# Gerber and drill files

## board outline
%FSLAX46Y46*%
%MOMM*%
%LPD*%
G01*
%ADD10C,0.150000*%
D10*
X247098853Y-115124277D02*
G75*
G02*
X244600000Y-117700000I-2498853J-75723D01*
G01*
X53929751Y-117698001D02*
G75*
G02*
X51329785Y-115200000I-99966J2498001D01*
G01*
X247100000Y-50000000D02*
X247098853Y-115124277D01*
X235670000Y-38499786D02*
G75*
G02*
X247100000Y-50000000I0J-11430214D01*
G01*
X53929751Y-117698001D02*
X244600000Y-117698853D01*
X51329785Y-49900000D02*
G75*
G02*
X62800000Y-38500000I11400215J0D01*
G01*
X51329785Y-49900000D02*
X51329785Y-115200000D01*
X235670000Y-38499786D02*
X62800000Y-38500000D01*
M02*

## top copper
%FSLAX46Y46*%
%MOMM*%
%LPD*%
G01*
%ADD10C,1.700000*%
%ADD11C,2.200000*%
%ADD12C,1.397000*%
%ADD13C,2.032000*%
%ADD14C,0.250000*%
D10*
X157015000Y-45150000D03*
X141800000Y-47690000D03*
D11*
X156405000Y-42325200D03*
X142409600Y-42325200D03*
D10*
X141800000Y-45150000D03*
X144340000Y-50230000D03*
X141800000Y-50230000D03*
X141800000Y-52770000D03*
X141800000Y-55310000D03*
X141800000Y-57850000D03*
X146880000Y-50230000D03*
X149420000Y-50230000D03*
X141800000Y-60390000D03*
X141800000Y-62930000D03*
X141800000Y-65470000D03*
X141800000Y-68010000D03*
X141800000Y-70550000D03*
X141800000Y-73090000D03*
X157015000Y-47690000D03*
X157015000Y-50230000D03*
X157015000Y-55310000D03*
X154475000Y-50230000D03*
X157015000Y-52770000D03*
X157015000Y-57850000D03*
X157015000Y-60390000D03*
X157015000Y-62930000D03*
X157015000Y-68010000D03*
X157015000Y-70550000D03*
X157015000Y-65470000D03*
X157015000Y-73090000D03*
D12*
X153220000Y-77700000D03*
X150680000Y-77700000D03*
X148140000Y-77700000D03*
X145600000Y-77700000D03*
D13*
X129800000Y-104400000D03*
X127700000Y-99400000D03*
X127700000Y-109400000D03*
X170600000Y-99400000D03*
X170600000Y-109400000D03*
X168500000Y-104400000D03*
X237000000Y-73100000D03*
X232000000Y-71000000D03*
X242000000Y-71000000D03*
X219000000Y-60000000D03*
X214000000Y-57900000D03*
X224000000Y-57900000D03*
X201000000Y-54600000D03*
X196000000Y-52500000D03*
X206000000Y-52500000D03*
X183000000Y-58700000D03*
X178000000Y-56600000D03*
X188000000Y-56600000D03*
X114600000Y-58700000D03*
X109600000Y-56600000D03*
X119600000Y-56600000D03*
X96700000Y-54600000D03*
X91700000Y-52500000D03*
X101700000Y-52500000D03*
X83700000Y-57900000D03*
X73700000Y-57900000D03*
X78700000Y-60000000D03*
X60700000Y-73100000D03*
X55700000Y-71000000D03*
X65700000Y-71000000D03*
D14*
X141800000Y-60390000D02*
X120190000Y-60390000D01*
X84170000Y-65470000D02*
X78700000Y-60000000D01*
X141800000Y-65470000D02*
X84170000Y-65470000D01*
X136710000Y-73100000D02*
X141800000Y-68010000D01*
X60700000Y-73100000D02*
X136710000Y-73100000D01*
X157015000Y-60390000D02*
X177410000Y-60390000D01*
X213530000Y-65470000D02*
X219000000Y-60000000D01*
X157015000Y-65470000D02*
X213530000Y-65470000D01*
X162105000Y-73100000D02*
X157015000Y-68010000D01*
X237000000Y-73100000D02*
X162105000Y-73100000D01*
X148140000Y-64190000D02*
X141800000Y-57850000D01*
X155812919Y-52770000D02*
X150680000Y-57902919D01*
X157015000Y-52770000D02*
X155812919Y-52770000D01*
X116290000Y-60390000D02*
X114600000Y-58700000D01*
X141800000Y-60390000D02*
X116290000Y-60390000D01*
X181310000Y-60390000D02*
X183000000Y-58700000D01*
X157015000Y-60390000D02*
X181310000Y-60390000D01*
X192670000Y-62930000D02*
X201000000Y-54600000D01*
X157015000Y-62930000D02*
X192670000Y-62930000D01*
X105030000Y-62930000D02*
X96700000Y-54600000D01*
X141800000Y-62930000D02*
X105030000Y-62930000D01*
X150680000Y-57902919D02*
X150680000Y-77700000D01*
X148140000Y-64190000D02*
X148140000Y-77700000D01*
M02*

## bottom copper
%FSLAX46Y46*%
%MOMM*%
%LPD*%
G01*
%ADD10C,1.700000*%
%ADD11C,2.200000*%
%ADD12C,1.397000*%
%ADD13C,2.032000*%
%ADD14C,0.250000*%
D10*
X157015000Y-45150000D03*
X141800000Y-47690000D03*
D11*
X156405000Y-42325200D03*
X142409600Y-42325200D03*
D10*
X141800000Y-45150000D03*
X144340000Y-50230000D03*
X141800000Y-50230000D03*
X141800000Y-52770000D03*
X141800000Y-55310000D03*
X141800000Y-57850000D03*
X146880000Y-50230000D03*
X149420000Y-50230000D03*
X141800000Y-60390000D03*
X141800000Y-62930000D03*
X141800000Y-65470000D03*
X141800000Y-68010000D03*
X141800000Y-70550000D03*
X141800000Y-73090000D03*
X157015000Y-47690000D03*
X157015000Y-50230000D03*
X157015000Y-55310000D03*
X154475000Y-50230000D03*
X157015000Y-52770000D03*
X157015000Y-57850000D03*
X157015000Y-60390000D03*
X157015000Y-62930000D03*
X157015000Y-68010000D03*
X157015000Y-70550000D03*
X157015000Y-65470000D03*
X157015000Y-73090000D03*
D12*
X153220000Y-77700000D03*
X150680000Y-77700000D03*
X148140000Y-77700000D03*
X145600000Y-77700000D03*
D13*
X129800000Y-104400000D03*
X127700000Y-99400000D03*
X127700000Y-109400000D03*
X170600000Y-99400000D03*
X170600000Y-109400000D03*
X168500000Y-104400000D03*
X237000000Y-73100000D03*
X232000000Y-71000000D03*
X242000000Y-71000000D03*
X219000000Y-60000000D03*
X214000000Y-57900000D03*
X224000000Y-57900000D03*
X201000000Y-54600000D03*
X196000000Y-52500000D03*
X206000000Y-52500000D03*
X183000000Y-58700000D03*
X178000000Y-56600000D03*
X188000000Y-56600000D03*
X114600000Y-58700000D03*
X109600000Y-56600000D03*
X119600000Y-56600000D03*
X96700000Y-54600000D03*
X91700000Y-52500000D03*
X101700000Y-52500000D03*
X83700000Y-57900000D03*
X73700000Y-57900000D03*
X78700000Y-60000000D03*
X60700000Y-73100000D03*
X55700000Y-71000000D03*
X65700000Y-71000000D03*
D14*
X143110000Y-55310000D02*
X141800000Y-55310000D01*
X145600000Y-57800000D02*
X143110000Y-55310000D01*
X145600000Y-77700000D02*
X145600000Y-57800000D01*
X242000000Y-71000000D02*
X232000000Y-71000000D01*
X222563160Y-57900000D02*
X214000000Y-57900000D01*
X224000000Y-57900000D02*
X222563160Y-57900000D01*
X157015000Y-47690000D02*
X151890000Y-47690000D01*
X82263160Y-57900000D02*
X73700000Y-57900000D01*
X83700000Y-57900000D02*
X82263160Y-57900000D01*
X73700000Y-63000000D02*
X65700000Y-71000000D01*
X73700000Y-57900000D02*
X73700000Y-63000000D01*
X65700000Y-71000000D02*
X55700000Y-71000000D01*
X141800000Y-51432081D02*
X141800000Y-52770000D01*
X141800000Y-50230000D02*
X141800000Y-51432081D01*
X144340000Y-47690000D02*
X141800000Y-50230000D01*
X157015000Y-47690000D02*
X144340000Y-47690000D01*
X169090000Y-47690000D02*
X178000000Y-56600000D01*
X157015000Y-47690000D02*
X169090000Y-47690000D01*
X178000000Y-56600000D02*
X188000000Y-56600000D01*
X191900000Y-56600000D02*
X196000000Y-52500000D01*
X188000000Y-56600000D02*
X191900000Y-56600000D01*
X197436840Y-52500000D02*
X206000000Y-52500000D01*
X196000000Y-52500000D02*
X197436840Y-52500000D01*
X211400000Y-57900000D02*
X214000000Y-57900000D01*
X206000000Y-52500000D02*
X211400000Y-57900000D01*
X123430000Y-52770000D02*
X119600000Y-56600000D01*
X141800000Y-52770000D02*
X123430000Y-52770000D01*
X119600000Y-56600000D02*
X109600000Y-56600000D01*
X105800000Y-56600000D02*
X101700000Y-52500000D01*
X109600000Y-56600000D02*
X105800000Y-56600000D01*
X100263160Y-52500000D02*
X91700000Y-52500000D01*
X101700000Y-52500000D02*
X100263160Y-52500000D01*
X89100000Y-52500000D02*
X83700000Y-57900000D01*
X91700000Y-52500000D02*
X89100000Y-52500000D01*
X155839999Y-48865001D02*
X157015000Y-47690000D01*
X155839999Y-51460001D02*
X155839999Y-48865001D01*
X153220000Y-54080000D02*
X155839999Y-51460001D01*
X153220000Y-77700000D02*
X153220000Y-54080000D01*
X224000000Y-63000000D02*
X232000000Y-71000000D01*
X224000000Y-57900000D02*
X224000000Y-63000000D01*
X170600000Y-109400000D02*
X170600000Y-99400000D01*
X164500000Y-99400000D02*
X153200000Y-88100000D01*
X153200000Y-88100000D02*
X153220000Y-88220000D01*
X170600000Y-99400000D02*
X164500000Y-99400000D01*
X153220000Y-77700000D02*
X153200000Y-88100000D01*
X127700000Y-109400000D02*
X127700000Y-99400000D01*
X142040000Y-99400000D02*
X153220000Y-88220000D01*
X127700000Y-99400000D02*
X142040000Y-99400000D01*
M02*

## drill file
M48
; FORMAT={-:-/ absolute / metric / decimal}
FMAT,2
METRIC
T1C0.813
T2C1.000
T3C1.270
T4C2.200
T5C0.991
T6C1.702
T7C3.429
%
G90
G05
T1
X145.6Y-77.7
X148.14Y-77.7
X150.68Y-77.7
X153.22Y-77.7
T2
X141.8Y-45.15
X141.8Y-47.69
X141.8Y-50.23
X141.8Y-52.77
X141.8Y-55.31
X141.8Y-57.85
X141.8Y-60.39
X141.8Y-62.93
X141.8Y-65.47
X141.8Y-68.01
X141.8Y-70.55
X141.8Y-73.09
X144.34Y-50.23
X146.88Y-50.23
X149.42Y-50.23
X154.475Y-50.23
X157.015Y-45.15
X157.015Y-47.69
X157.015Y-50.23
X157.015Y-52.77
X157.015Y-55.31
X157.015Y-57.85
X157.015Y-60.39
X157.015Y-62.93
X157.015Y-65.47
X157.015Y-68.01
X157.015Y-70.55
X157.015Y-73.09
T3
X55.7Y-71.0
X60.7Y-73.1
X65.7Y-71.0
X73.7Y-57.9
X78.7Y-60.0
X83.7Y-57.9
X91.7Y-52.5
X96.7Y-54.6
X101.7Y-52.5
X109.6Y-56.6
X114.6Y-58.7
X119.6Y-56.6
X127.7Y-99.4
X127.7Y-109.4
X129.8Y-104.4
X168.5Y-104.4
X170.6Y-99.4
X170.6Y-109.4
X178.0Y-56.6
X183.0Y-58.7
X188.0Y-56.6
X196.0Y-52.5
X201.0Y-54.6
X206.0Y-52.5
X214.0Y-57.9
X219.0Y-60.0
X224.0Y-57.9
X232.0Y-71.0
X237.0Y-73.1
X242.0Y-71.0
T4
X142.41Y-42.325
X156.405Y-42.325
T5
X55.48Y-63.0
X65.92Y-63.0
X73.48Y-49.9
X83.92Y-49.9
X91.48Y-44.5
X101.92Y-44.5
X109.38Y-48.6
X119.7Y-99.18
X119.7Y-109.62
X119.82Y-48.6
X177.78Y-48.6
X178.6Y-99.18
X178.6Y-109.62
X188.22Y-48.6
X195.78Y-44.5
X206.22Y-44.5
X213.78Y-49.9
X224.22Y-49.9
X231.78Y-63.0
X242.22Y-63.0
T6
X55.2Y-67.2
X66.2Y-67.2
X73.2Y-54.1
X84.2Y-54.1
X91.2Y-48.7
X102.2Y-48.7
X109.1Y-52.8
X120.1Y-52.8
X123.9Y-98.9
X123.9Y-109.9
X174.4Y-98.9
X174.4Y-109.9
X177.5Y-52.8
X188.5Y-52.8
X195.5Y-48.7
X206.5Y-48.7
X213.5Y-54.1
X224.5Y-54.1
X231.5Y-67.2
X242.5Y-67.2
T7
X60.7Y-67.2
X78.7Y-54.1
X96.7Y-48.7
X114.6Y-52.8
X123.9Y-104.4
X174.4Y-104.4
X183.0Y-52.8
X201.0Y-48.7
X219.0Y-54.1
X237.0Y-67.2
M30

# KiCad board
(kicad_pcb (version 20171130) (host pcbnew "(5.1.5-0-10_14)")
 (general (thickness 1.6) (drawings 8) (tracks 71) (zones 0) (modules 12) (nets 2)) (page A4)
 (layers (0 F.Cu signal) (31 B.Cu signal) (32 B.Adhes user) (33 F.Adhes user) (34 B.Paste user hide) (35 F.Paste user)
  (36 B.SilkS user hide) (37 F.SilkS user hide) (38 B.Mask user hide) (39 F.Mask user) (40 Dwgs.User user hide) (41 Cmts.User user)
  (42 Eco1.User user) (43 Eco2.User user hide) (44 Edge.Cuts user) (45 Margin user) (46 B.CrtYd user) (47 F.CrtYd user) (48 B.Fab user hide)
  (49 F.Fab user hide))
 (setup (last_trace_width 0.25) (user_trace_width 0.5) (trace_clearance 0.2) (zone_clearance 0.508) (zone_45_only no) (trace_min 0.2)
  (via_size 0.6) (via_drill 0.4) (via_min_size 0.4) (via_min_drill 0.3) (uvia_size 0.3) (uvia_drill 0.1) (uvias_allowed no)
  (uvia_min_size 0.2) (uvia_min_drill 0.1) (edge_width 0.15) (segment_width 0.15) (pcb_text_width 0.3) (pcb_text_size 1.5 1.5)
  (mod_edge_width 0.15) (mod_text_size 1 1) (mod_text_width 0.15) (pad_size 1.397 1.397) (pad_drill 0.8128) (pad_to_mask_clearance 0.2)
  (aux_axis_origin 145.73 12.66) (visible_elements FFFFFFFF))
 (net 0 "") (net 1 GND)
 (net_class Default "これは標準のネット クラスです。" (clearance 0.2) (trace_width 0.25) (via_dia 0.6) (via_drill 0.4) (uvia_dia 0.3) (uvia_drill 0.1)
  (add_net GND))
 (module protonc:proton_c (layer F.Cu) (at 149.4 60.4)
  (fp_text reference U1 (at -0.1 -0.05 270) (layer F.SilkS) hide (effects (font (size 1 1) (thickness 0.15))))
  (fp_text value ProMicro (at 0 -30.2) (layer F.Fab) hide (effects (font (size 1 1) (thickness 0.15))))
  (pad 5V thru_hole circle (at 7.615 -15.25) (size 1.7 1.7) (drill 1) (layers *.Cu *.Mask))
  (pad A10 thru_hole circle (at -7.6 -12.71) (size 1.7 1.7) (drill 1) (layers *.Cu *.Mask))
  (pad SCRE thru_hole circle (at 7.005 -18.0748) (size 2.2 2.2) (drill 2.2) (layers *.Cu *.Mask))
  (pad SCRE thru_hole circle (at -6.9904 -18.0748) (size 2.2 2.2) (drill 2.2) (layers *.Cu *.Mask))
  (pad A9 thru_hole circle (at -7.6 -15.25) (size 1.7 1.7) (drill 1) (layers *.Cu *.Mask))
  (pad D+ thru_hole circle (at -5.06 -10.17) (size 1.7 1.7) (drill 1) (layers *.Cu *.Mask))
  (pad GND thru_hole circle (at -7.6 -10.17) (size 1.7 1.7) (drill 1) (layers *.Cu *.Mask) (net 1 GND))
  (pad GND thru_hole circle (at -7.6 -7.63) (size 1.7 1.7) (drill 1) (layers *.Cu *.Mask) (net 1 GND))
  (pad B7 thru_hole circle (at -7.6 -5.09) (size 1.7 1.7) (drill 1) (layers *.Cu *.Mask))
  (pad B6 thru_hole circle (at -7.6 -2.55) (size 1.7 1.7) (drill 1) (layers *.Cu *.Mask))
  (pad D- thru_hole circle (at -2.52 -10.17) (size 1.7 1.7) (drill 1) (layers *.Cu *.Mask))
  (pad CHRG thru_hole circle (at 0.02 -10.17) (size 1.7 1.7) (drill 1) (layers *.Cu *.Mask))
  (pad B5 thru_hole circle (at -7.6 -0.01) (size 1.7 1.7) (drill 1) (layers *.Cu *.Mask))
  (pad B4 thru_hole circle (at -7.6 2.53) (size 1.7 1.7) (drill 1) (layers *.Cu *.Mask))
  (pad B3 thru_hole circle (at -7.6 5.07) (size 1.7 1.7) (drill 1) (layers *.Cu *.Mask))
  (pad B2 thru_hole circle (at -7.6 7.61) (size 1.7 1.7) (drill 1) (layers *.Cu *.Mask))
  (pad B1 thru_hole circle (at -7.6 10.15) (size 1.7 1.7) (drill 1) (layers *.Cu *.Mask))
  (pad B0 thru_hole circle (at -7.6 12.69) (size 1.7 1.7) (drill 1) (layers *.Cu *.Mask))
  (pad GND thru_hole circle (at 7.615 -12.71) (size 1.7 1.7) (drill 1) (layers *.Cu *.Mask) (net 1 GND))
  (pad DFU thru_hole circle (at 7.615 -10.17) (size 1.7 1.7) (drill 1) (layers *.Cu *.Mask))
  (pad A2 thru_hole circle (at 7.615 -5.09) (size 1.7 1.7) (drill 1) (layers *.Cu *.Mask))
  (pad A3|5v thru_hole circle (at 5.075 -10.17) (size 1.7 1.7) (drill 1) (layers *.Cu *.Mask))
  (pad 3.3V thru_hole circle (at 7.615 -7.63) (size 1.7 1.7) (drill 1) (layers *.Cu *.Mask))
  (pad A1 thru_hole circle (at 7.615 -2.55) (size 1.7 1.7) (drill 1) (layers *.Cu *.Mask))
  (pad A0 thru_hole circle (at 7.615 -0.01) (size 1.7 1.7) (drill 1) (layers *.Cu *.Mask))
  (pad B8 thru_hole circle (at 7.615 2.53) (size 1.7 1.7) (drill 1) (layers *.Cu *.Mask))
  (pad B14 thru_hole circle (at 7.615 7.61) (size 1.7 1.7) (drill 1) (layers *.Cu *.Mask))
  (pad B15 thru_hole circle (at 7.615 10.15) (size 1.7 1.7) (drill 1) (layers *.Cu *.Mask))
  (pad B13 thru_hole circle (at 7.615 5.07) (size 1.7 1.7) (drill 1) (layers *.Cu *.Mask))
  (pad B9 thru_hole circle (at 7.615 12.69) (size 1.7 1.7) (drill 1) (layers *.Cu *.Mask)))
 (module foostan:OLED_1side (layer F.Cu) (at 145.6 77.7)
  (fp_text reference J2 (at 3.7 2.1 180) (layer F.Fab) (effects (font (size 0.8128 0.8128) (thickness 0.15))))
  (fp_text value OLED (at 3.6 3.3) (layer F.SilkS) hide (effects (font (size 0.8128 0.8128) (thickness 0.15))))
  (pad 4 thru_hole circle (at 7.62 0) (size 1.397 1.397) (drill 0.8128) (layers *.Cu F.SilkS B.Mask) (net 1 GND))
  (pad 3 thru_hole circle (at 5.08 0) (size 1.397 1.397) (drill 0.8128) (layers *.Cu F.SilkS B.Mask))
  (pad 2 thru_hole circle (at 2.54 0) (size 1.397 1.397) (drill 0.8128) (layers *.Cu F.SilkS B.Mask))
  (pad 1 thru_hole circle (at 0 0) (size 1.397 1.397) (drill 0.8128) (layers *.Cu F.SilkS B.Mask)))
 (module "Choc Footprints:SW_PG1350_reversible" (layer B.Cu) (at 123.9 104.4 270)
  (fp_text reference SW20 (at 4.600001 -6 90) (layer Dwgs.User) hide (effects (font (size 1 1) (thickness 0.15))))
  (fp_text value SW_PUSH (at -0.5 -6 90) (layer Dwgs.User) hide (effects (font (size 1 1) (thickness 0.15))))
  (pad "" np_thru_hole circle (at -5.5 0 270) (size 1.7018 1.7018) (drill 1.7018) (layers *.Cu *.Mask))
  (pad "" np_thru_hole circle (at 5.5 0 270) (size 1.7018 1.7018) (drill 1.7018) (layers *.Cu *.Mask))
  (pad "" np_thru_hole circle (at 5.22 4.2 270) (size 0.9906 0.9906) (drill 0.9906) (layers *.Cu *.Mask))
  (pad 1 thru_hole circle (at 0 -5.9 270) (size 2.032 2.032) (drill 1.27) (layers *.Cu *.Mask))
  (pad 2 thru_hole circle (at -5 -3.8 270) (size 2.032 2.032) (drill 1.27) (layers *.Cu *.Mask) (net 1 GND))
  (pad "" np_thru_hole circle (at 0 0 270) (size 3.429 3.429) (drill 3.429) (layers *.Cu *.Mask))
  (pad 2 thru_hole circle (at 5 -3.8 270) (size 2.032 2.032) (drill 1.27) (layers *.Cu *.Mask) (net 1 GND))
  (pad "" np_thru_hole circle (at -5.22 4.2 270) (size 0.9906 0.9906) (drill 0.9906) (layers *.Cu *.Mask)))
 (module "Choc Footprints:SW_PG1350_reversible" (layer B.Cu) (at 174.4 104.4 90)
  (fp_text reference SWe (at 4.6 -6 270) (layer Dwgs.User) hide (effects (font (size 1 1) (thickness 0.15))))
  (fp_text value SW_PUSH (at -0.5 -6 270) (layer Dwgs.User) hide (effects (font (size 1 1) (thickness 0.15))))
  (pad "" np_thru_hole circle (at -5.22 4.2 90) (size 0.9906 0.9906) (drill 0.9906) (layers *.Cu *.Mask))
  (pad 2 thru_hole circle (at 5 -3.8 90) (size 2.032 2.032) (drill 1.27) (layers *.Cu *.Mask) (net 1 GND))
  (pad "" np_thru_hole circle (at 0 0 90) (size 3.429 3.429) (drill 3.429) (layers *.Cu *.Mask))
  (pad 2 thru_hole circle (at -5 -3.8 90) (size 2.032 2.032) (drill 1.27) (layers *.Cu *.Mask) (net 1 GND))
  (pad 1 thru_hole circle (at 0 -5.9 90) (size 2.032 2.032) (drill 1.27) (layers *.Cu *.Mask))
  (pad "" np_thru_hole circle (at 5.22 4.2 90) (size 0.9906 0.9906) (drill 0.9906) (layers *.Cu *.Mask))
  (pad "" np_thru_hole circle (at 5.5 0 90) (size 1.7018 1.7018) (drill 1.7018) (layers *.Cu *.Mask))
  (pad "" np_thru_hole circle (at -5.5 0 90) (size 1.7018 1.7018) (drill 1.7018) (layers *.Cu *.Mask)))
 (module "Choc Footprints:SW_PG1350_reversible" (layer F.Cu) (at 237 67.2)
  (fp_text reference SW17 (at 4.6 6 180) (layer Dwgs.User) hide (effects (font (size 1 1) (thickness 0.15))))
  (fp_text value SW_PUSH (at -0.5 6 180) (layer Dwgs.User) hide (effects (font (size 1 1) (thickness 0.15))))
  (pad "" np_thru_hole circle (at -5.5 0) (size 1.7018 1.7018) (drill 1.7018) (layers *.Cu *.Mask))
  (pad "" np_thru_hole circle (at 5.5 0) (size 1.7018 1.7018) (drill 1.7018) (layers *.Cu *.Mask))
  (pad "" np_thru_hole circle (at 5.22 -4.2) (size 0.9906 0.9906) (drill 0.9906) (layers *.Cu *.Mask))
  (pad 1 thru_hole circle (at 0 5.9) (size 2.032 2.032) (drill 1.27) (layers *.Cu *.Mask))
  (pad 2 thru_hole circle (at -5 3.8) (size 2.032 2.032) (drill 1.27) (layers *.Cu *.Mask) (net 1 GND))
  (pad "" np_thru_hole circle (at 0 0) (size 3.429 3.429) (drill 3.429) (layers *.Cu *.Mask))
  (pad 2 thru_hole circle (at 5 3.8) (size 2.032 2.032) (drill 1.27) (layers *.Cu *.Mask) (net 1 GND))
  (pad "" np_thru_hole circle (at -5.22 -4.2) (size 0.9906 0.9906) (drill 0.9906) (layers *.Cu *.Mask)))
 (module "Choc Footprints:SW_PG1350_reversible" (layer F.Cu) (at 219 54.1)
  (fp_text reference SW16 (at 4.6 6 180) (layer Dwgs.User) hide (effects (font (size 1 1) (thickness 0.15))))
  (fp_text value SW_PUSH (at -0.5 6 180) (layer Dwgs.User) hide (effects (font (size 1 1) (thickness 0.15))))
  (pad "" np_thru_hole circle (at -5.5 0) (size 1.7018 1.7018) (drill 1.7018) (layers *.Cu *.Mask))
  (pad "" np_thru_hole circle (at 5.5 0) (size 1.7018 1.7018) (drill 1.7018) (layers *.Cu *.Mask))
  (pad "" np_thru_hole circle (at 5.22 -4.2) (size 0.9906 0.9906) (drill 0.9906) (layers *.Cu *.Mask))
  (pad 1 thru_hole circle (at 0 5.9) (size 2.032 2.032) (drill 1.27) (layers *.Cu *.Mask))
  (pad 2 thru_hole circle (at -5 3.8) (size 2.032 2.032) (drill 1.27) (layers *.Cu *.Mask) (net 1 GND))
  (pad "" np_thru_hole circle (at 0 0) (size 3.429 3.429) (drill 3.429) (layers *.Cu *.Mask))
  (pad 2 thru_hole circle (at 5 3.8) (size 2.032 2.032) (drill 1.27) (layers *.Cu *.Mask) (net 1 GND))
  (pad "" np_thru_hole circle (at -5.22 -4.2) (size 0.9906 0.9906) (drill 0.9906) (layers *.Cu *.Mask)))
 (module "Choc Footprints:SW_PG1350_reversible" (layer F.Cu) (at 201 48.7)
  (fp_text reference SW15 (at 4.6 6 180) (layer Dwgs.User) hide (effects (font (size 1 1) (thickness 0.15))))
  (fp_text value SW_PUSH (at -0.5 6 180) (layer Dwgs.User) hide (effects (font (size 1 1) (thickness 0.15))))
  (pad "" np_thru_hole circle (at -5.5 0) (size 1.7018 1.7018) (drill 1.7018) (layers *.Cu *.Mask))
  (pad "" np_thru_hole circle (at 5.5 0) (size 1.7018 1.7018) (drill 1.7018) (layers *.Cu *.Mask))
  (pad "" np_thru_hole circle (at 5.22 -4.2) (size 0.9906 0.9906) (drill 0.9906) (layers *.Cu *.Mask))
  (pad 1 thru_hole circle (at 0 5.9) (size 2.032 2.032) (drill 1.27) (layers *.Cu *.Mask))
  (pad 2 thru_hole circle (at -5 3.8) (size 2.032 2.032) (drill 1.27) (layers *.Cu *.Mask) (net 1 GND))
  (pad "" np_thru_hole circle (at 0 0) (size 3.429 3.429) (drill 3.429) (layers *.Cu *.Mask))
  (pad 2 thru_hole circle (at 5 3.8) (size 2.032 2.032) (drill 1.27) (layers *.Cu *.Mask) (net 1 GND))
  (pad "" np_thru_hole circle (at -5.22 -4.2) (size 0.9906 0.9906) (drill 0.9906) (layers *.Cu *.Mask)))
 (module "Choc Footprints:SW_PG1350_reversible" (layer F.Cu) (at 183 52.8)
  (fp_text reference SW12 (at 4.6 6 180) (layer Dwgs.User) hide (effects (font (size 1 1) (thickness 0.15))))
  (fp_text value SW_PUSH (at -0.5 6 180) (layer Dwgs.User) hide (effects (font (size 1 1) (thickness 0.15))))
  (pad "" np_thru_hole circle (at -5.5 0) (size 1.7018 1.7018) (drill 1.7018) (layers *.Cu *.Mask))
  (pad "" np_thru_hole circle (at 5.5 0) (size 1.7018 1.7018) (drill 1.7018) (layers *.Cu *.Mask))
  (pad "" np_thru_hole circle (at 5.22 -4.2) (size 0.9906 0.9906) (drill 0.9906) (layers *.Cu *.Mask))
  (pad 1 thru_hole circle (at 0 5.9) (size 2.032 2.032) (drill 1.27) (layers *.Cu *.Mask))
  (pad 2 thru_hole circle (at -5 3.8) (size 2.032 2.032) (drill 1.27) (layers *.Cu *.Mask) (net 1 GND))
  (pad "" np_thru_hole circle (at 0 0) (size 3.429 3.429) (drill 3.429) (layers *.Cu *.Mask))
  (pad 2 thru_hole circle (at 5 3.8) (size 2.032 2.032) (drill 1.27) (layers *.Cu *.Mask) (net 1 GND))
  (pad "" np_thru_hole circle (at -5.22 -4.2) (size 0.9906 0.9906) (drill 0.9906) (layers *.Cu *.Mask)))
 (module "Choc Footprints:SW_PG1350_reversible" (layer F.Cu) (at 114.6 52.8)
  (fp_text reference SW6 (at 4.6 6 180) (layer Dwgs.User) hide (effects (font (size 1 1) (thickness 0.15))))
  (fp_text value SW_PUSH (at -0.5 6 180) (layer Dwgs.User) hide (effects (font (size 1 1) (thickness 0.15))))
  (pad "" np_thru_hole circle (at -5.5 0) (size 1.7018 1.7018) (drill 1.7018) (layers *.Cu *.Mask))
  (pad "" np_thru_hole circle (at 5.5 0) (size 1.7018 1.7018) (drill 1.7018) (layers *.Cu *.Mask))
  (pad "" np_thru_hole circle (at 5.22 -4.2) (size 0.9906 0.9906) (drill 0.9906) (layers *.Cu *.Mask))
  (pad 1 thru_hole circle (at 0 5.9) (size 2.032 2.032) (drill 1.27) (layers *.Cu *.Mask))
  (pad 2 thru_hole circle (at -5 3.8) (size 2.032 2.032) (drill 1.27) (layers *.Cu *.Mask) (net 1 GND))
  (pad "" np_thru_hole circle (at 0 0) (size 3.429 3.429) (drill 3.429) (layers *.Cu *.Mask))
  (pad 2 thru_hole circle (at 5 3.8) (size 2.032 2.032) (drill 1.27) (layers *.Cu *.Mask) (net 1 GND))
  (pad "" np_thru_hole circle (at -5.22 -4.2) (size 0.9906 0.9906) (drill 0.9906) (layers *.Cu *.Mask)))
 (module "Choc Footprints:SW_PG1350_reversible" (layer F.Cu) (at 96.7 48.7)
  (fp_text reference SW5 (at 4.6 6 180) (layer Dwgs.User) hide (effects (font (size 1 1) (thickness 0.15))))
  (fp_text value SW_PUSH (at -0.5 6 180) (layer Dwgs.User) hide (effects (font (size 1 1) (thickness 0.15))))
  (pad "" np_thru_hole circle (at -5.5 0) (size 1.7018 1.7018) (drill 1.7018) (layers *.Cu *.Mask))
  (pad "" np_thru_hole circle (at 5.5 0) (size 1.7018 1.7018) (drill 1.7018) (layers *.Cu *.Mask))
  (pad "" np_thru_hole circle (at 5.22 -4.2) (size 0.9906 0.9906) (drill 0.9906) (layers *.Cu *.Mask))
  (pad 1 thru_hole circle (at 0 5.9) (size 2.032 2.032) (drill 1.27) (layers *.Cu *.Mask))
  (pad 2 thru_hole circle (at -5 3.8) (size 2.032 2.032) (drill 1.27) (layers *.Cu *.Mask) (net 1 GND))
  (pad "" np_thru_hole circle (at 0 0) (size 3.429 3.429) (drill 3.429) (layers *.Cu *.Mask))
  (pad 2 thru_hole circle (at 5 3.8) (size 2.032 2.032) (drill 1.27) (layers *.Cu *.Mask) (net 1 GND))
  (pad "" np_thru_hole circle (at -5.22 -4.2) (size 0.9906 0.9906) (drill 0.9906) (layers *.Cu *.Mask)))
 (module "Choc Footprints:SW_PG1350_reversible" (layer F.Cu) (at 78.7 54.1)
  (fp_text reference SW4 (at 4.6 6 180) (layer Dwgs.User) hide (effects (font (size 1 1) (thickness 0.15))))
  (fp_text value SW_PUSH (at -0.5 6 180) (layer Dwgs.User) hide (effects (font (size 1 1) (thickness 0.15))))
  (pad "" np_thru_hole circle (at -5.22 -4.2) (size 0.9906 0.9906) (drill 0.9906) (layers *.Cu *.Mask))
  (pad 2 thru_hole circle (at 5 3.8) (size 2.032 2.032) (drill 1.27) (layers *.Cu *.Mask) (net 1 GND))
  (pad "" np_thru_hole circle (at 0 0) (size 3.429 3.429) (drill 3.429) (layers *.Cu *.Mask))
  (pad 2 thru_hole circle (at -5 3.8) (size 2.032 2.032) (drill 1.27) (layers *.Cu *.Mask) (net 1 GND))
  (pad 1 thru_hole circle (at 0 5.9) (size 2.032 2.032) (drill 1.27) (layers *.Cu *.Mask))
  (pad "" np_thru_hole circle (at 5.22 -4.2) (size 0.9906 0.9906) (drill 0.9906) (layers *.Cu *.Mask))
  (pad "" np_thru_hole circle (at 5.5 0) (size 1.7018 1.7018) (drill 1.7018) (layers *.Cu *.Mask))
  (pad "" np_thru_hole circle (at -5.5 0) (size 1.7018 1.7018) (drill 1.7018) (layers *.Cu *.Mask)))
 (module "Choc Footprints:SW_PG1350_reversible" (layer F.Cu) (at 60.7 67.2)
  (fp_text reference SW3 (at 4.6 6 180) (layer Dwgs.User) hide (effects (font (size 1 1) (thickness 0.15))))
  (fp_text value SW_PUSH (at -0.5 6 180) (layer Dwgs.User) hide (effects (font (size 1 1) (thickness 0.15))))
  (pad "" np_thru_hole circle (at -5.5 0) (size 1.7018 1.7018) (drill 1.7018) (layers *.Cu *.Mask))
  (pad "" np_thru_hole circle (at 5.5 0) (size 1.7018 1.7018) (drill 1.7018) (layers *.Cu *.Mask))
  (pad "" np_thru_hole circle (at 5.22 -4.2) (size 0.9906 0.9906) (drill 0.9906) (layers *.Cu *.Mask))
  (pad 1 thru_hole circle (at 0 5.9) (size 2.032 2.032) (drill 1.27) (layers *.Cu *.Mask))
  (pad 2 thru_hole circle (at -5 3.8) (size 2.032 2.032) (drill 1.27) (layers *.Cu *.Mask) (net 1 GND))
  (pad "" np_thru_hole circle (at 0 0) (size 3.429 3.429) (drill 3.429) (layers *.Cu *.Mask))
  (pad 2 thru_hole circle (at 5 3.8) (size 2.032 2.032) (drill 1.27) (layers *.Cu *.Mask) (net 1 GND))
  (pad "" np_thru_hole circle (at -5.22 -4.2) (size 0.9906 0.9906) (drill 0.9906) (layers *.Cu *.Mask)))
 (gr_arc (start 244.6 115.2) (end 244.6 117.7) (angle -91.73570459) (layer Edge.Cuts) (width 0.15))
 (gr_arc (start 53.829785 115.2) (end 51.329785 115.2) (angle -92.29166034) (layer Edge.Cuts) (width 0.15))
 (gr_line (start 247.1 50) (end 247.098853 115.124277) (angle 90) (layer Edge.Cuts) (width 0.15))
 (gr_arc (start 235.67 49.93) (end 247.1 50) (angle -90.3508884) (layer Edge.Cuts) (width 0.15))
 (gr_line (start 53.929751 117.698001) (end 244.6 117.698853) (angle 90) (layer Edge.Cuts) (width 0.15))
 (gr_arc (start 62.73 49.9) (end 62.8 38.5) (angle -90.35181177) (layer Edge.Cuts) (width 0.15))
 (gr_line (start 51.329785 49.9) (end 51.329785 115.2) (angle 90) (layer Edge.Cuts) (width 0.15))
 (gr_line (start 235.67 38.499786) (end 62.8 38.5) (angle 90) (layer Edge.Cuts) (width 0.15))
 (segment (start 141.8 60.39) (end 120.19 60.39) (width 0.25) (layer F.Cu) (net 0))
 (segment (start 84.17 65.47) (end 78.7 60) (width 0.25) (layer F.Cu) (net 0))
 (segment (start 141.8 65.47) (end 84.17 65.47) (width 0.25) (layer F.Cu) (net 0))
 (segment (start 136.71 73.1) (end 141.8 68.01) (width 0.25) (layer F.Cu) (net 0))
 (segment (start 60.7 73.1) (end 136.71 73.1) (width 0.25) (layer F.Cu) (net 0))
 (segment (start 157.015 60.39) (end 177.41 60.39) (width 0.25) (layer F.Cu) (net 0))
 (segment (start 213.53 65.47) (end 219 60) (width 0.25) (layer F.Cu) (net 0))
 (segment (start 157.015 65.47) (end 213.53 65.47) (width 0.25) (layer F.Cu) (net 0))
 (segment (start 162.105 73.1) (end 157.015 68.01) (width 0.25) (layer F.Cu) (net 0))
 (segment (start 237 73.1) (end 162.105 73.1) (width 0.25) (layer F.Cu) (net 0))
 (segment (start 148.14 64.19) (end 141.8 57.85) (width 0.25) (layer F.Cu) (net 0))
 (segment (start 155.812919 52.77) (end 150.68 57.902919) (width 0.25) (layer F.Cu) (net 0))
 (segment (start 157.015 52.77) (end 155.812919 52.77) (width 0.25) (layer F.Cu) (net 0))
 (segment (start 116.29 60.39) (end 114.6 58.7) (width 0.25) (layer F.Cu) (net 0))
 (segment (start 141.8 60.39) (end 116.29 60.39) (width 0.25) (layer F.Cu) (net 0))
 (segment (start 181.31 60.39) (end 183 58.7) (width 0.25) (layer F.Cu) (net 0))
 (segment (start 157.015 60.39) (end 181.31 60.39) (width 0.25) (layer F.Cu) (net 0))
 (segment (start 192.67 62.93) (end 201 54.6) (width 0.25) (layer F.Cu) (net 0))
 (segment (start 157.015 62.93) (end 192.67 62.93) (width 0.25) (layer F.Cu) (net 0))
 (segment (start 105.03 62.93) (end 96.7 54.6) (width 0.25) (layer F.Cu) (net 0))
 (segment (start 141.8 62.93) (end 105.03 62.93) (width 0.25) (layer F.Cu) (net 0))
 (segment (start 143.11 55.31) (end 141.8 55.31) (width 0.25) (layer B.Cu) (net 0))
 (segment (start 145.6 57.8) (end 143.11 55.31) (width 0.25) (layer B.Cu) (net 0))
 (segment (start 145.6 77.7) (end 145.6 57.8) (width 0.25) (layer B.Cu) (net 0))
 (segment (start 150.68 57.902919) (end 150.68 77.7) (width 0.25) (layer F.Cu) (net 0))
 (segment (start 148.14 64.19) (end 148.14 77.7) (width 0.25) (layer F.Cu) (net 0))
 (segment (start 242 71) (end 232 71) (width 0.25) (layer B.Cu) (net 1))
 (segment (start 222.56316 57.9) (end 214 57.9) (width 0.25) (layer B.Cu) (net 1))
 (segment (start 224 57.9) (end 222.56316 57.9) (width 0.25) (layer B.Cu) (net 1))
 (segment (start 157.015 47.69) (end 151.89 47.69) (width 0.25) (layer B.Cu) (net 1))
 (segment (start 82.26316 57.9) (end 73.7 57.9) (width 0.25) (layer B.Cu) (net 1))
 (segment (start 83.7 57.9) (end 82.26316 57.9) (width 0.25) (layer B.Cu) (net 1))
 (segment (start 73.7 63) (end 65.7 71) (width 0.25) (layer B.Cu) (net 1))
 (segment (start 73.7 57.9) (end 73.7 63) (width 0.25) (layer B.Cu) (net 1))
 (segment (start 65.7 71) (end 55.7 71) (width 0.25) (layer B.Cu) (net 1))
 (segment (start 141.8 51.432081) (end 141.8 52.77) (width 0.25) (layer B.Cu) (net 1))
 (segment (start 141.8 50.23) (end 141.8 51.432081) (width 0.25) (layer B.Cu) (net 1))
 (segment (start 144.34 47.69) (end 141.8 50.23) (width 0.25) (layer B.Cu) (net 1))
 (segment (start 157.015 47.69) (end 144.34 47.69) (width 0.25) (layer B.Cu) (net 1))
 (segment (start 169.09 47.69) (end 178 56.6) (width 0.25) (layer B.Cu) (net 1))
 (segment (start 157.015 47.69) (end 169.09 47.69) (width 0.25) (layer B.Cu) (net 1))
 (segment (start 178 56.6) (end 188 56.6) (width 0.25) (layer B.Cu) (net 1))
 (segment (start 191.9 56.6) (end 196 52.5) (width 0.25) (layer B.Cu) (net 1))
 (segment (start 188 56.6) (end 191.9 56.6) (width 0.25) (layer B.Cu) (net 1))
 (segment (start 197.43684 52.5) (end 206 52.5) (width 0.25) (layer B.Cu) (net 1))
 (segment (start 196 52.5) (end 197.43684 52.5) (width 0.25) (layer B.Cu) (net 1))
 (segment (start 211.4 57.9) (end 214 57.9) (width 0.25) (layer B.Cu) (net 1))
 (segment (start 206 52.5) (end 211.4 57.9) (width 0.25) (layer B.Cu) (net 1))
 (segment (start 123.43 52.77) (end 119.6 56.6) (width 0.25) (layer B.Cu) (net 1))
 (segment (start 141.8 52.77) (end 123.43 52.77) (width 0.25) (layer B.Cu) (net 1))
 (segment (start 119.6 56.6) (end 109.6 56.6) (width 0.25) (layer B.Cu) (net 1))
 (segment (start 105.8 56.6) (end 101.7 52.5) (width 0.25) (layer B.Cu) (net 1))
 (segment (start 109.6 56.6) (end 105.8 56.6) (width 0.25) (layer B.Cu) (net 1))
 (segment (start 100.26316 52.5) (end 91.7 52.5) (width 0.25) (layer B.Cu) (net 1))
 (segment (start 101.7 52.5) (end 100.26316 52.5) (width 0.25) (layer B.Cu) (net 1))
 (segment (start 89.1 52.5) (end 83.7 57.9) (width 0.25) (layer B.Cu) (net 1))
 (segment (start 91.7 52.5) (end 89.1 52.5) (width 0.25) (layer B.Cu) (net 1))
 (segment (start 155.839999 48.865001) (end 157.015 47.69) (width 0.25) (layer B.Cu) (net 1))
 (segment (start 155.839999 51.460001) (end 155.839999 48.865001) (width 0.25) (layer B.Cu) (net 1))
 (segment (start 153.22 54.08) (end 155.839999 51.460001) (width 0.25) (layer B.Cu) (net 1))
 (segment (start 153.22 77.7) (end 153.22 54.08) (width 0.25) (layer B.Cu) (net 1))
 (segment (start 224 63) (end 232 71) (width 0.25) (layer B.Cu) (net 1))
 (segment (start 224 57.9) (end 224 63) (width 0.25) (layer B.Cu) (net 1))
 (segment (start 170.6 109.4) (end 170.6 99.4) (width 0.25) (layer B.Cu) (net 1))
 (segment (start 164.5 99.4) (end 153.2 88.1) (width 0.25) (layer B.Cu) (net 1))
 (segment (start 153.2 88.1) (end 153.22 88.22) (width 0.25) (layer B.Cu) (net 1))
 (segment (start 170.6 99.4) (end 164.5 99.4) (width 0.25) (layer B.Cu) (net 1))
 (segment (start 153.22 77.7) (end 153.2 88.1) (width 0.25) (layer B.Cu) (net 1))
 (segment (start 127.7 109.4) (end 127.7 99.4) (width 0.25) (layer B.Cu) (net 1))
 (segment (start 142.04 99.4) (end 153.22 88.22) (width 0.25) (layer B.Cu) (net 1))
 (segment (start 127.7 99.4) (end 142.04 99.4) (width 0.25) (layer B.Cu) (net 1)))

